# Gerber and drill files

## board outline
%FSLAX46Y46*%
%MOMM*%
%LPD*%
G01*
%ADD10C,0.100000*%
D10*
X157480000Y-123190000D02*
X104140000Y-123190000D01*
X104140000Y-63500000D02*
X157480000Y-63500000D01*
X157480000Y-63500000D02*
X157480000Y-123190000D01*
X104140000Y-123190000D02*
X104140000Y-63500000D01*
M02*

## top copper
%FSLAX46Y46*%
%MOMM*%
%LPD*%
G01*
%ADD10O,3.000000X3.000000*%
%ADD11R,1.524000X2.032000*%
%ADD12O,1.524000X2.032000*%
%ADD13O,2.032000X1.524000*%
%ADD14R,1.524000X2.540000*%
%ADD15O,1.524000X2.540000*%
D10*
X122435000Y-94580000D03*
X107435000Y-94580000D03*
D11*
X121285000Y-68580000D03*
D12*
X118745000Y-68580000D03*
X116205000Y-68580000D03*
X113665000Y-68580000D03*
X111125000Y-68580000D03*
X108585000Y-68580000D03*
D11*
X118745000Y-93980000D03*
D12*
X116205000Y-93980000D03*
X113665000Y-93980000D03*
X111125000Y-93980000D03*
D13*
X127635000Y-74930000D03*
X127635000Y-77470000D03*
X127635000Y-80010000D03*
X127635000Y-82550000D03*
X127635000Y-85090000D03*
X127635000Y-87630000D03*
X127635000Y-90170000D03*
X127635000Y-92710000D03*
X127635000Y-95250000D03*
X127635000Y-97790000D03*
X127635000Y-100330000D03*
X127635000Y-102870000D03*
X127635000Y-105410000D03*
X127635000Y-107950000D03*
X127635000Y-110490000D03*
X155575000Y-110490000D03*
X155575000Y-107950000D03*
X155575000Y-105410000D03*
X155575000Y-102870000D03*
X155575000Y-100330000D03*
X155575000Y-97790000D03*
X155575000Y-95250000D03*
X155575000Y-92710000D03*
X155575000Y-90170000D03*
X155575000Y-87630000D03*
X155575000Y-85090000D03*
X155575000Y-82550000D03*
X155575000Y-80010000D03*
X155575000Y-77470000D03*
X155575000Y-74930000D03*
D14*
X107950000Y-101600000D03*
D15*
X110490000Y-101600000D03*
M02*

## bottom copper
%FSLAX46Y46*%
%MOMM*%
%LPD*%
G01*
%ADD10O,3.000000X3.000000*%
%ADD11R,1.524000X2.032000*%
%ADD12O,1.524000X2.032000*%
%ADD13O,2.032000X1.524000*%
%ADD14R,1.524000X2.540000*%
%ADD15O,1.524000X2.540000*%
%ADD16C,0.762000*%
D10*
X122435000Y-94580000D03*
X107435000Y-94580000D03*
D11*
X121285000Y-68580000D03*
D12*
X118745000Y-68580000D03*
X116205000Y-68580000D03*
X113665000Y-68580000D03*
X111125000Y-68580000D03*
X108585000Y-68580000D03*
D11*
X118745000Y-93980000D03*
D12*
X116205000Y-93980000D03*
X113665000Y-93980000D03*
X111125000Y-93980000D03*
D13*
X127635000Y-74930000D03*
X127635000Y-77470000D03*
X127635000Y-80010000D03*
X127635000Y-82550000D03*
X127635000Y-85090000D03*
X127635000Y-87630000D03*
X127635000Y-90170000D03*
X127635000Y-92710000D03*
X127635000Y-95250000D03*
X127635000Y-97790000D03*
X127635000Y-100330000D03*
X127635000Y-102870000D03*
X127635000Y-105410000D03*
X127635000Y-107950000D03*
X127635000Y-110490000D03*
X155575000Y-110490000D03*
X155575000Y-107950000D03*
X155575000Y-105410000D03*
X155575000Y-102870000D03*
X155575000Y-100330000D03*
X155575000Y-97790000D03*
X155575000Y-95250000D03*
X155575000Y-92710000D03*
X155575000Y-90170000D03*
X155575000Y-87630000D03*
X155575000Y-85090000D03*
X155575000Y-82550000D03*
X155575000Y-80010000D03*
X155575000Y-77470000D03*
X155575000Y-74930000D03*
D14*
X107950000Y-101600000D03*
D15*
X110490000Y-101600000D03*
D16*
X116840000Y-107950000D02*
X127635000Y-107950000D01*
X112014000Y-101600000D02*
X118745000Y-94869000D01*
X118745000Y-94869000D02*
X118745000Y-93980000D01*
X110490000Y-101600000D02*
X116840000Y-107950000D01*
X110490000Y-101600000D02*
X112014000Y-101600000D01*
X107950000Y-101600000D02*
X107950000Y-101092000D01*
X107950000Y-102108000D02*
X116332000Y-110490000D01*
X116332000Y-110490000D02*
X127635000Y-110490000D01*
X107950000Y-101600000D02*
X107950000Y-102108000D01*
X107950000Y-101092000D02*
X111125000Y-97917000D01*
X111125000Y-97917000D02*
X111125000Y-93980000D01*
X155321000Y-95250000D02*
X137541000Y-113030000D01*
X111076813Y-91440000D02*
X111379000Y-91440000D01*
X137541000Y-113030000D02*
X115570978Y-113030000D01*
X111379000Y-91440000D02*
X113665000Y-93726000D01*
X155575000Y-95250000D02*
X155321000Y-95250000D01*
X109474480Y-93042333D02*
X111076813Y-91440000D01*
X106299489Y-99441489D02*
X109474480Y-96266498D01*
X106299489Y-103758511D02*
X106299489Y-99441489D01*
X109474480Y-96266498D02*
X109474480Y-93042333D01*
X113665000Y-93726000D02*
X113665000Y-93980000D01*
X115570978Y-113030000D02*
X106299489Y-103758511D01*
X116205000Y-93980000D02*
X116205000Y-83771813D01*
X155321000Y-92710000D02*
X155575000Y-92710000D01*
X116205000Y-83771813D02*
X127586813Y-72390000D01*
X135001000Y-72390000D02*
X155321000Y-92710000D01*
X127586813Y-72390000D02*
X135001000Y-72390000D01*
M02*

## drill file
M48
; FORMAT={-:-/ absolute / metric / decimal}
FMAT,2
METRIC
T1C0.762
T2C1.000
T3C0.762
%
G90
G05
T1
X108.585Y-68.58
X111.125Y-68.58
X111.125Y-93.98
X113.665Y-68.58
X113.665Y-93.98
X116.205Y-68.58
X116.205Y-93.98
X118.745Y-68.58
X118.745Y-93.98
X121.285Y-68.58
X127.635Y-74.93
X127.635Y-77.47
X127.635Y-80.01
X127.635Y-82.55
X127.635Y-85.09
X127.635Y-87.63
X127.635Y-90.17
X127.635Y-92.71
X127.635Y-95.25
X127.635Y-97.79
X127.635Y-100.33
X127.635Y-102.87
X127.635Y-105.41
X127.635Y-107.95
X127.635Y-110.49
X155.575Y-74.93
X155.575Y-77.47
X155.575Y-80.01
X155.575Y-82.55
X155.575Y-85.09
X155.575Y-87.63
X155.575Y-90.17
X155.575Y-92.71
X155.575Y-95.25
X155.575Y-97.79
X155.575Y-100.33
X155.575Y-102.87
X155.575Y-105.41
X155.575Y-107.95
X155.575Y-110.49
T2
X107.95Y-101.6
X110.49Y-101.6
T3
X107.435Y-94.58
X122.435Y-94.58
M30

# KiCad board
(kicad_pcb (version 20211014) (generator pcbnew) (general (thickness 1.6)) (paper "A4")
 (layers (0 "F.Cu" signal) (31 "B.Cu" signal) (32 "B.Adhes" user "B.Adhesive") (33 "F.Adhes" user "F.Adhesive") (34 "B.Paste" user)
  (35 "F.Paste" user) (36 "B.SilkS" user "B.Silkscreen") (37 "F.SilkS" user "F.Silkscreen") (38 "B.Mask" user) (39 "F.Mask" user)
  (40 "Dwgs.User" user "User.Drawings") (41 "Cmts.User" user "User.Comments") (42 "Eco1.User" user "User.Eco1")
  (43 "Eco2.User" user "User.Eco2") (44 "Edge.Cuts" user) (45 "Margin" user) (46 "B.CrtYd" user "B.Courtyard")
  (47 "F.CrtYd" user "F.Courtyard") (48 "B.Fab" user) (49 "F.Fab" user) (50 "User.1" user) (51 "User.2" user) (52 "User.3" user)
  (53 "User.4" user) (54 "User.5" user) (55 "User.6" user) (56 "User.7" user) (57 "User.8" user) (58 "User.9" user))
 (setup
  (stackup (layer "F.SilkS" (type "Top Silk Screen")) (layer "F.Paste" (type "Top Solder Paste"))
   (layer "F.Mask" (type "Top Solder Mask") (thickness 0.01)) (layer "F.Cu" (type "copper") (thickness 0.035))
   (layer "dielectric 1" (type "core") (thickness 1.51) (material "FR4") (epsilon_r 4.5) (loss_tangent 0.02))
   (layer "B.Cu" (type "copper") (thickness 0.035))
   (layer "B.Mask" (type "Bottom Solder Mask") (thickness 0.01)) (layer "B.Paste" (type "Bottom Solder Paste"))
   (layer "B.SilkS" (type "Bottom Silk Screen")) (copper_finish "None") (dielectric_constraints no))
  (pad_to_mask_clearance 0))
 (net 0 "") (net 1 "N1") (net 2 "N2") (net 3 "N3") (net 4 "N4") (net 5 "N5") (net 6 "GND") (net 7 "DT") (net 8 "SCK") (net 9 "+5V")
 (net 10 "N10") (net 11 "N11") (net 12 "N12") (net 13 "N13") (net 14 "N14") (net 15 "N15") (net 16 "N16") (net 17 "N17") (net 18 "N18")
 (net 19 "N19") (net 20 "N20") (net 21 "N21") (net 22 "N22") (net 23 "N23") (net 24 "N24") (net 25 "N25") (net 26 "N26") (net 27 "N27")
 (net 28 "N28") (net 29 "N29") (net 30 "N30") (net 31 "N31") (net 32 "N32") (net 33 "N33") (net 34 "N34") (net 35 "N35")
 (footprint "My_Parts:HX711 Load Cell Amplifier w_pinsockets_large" (layer "F.Cu") (at 114.935 68.58 -90)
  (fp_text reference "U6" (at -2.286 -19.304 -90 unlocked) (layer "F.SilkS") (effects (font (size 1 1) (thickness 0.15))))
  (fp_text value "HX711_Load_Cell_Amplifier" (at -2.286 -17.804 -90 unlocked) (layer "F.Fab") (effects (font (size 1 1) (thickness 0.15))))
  (pad "" np_thru_hole oval (at 26 -7.5 270) (size 3 3) (drill 0.762) (layers F&B.Cu *.Mask))
  (pad "" np_thru_hole oval (at 26 7.5 270) (size 3 3) (drill 0.762) (layers F&B.Cu *.Mask))
  (pad "1" thru_hole rect (at 0 -6.35 270) (size 2.032 1.524) (drill 0.762) (layers *.Cu *.Mask) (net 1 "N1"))
  (pad "2" thru_hole oval (at 0 -3.81 270) (size 2.032 1.524) (drill 0.762) (layers *.Cu *.Mask) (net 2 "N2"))
  (pad "3" thru_hole oval (at 0 -1.27 270) (size 2.032 1.524) (drill 0.762) (layers *.Cu *.Mask))
  (pad "4" thru_hole oval (at 0 1.27 270) (size 2.032 1.524) (drill 0.762) (layers *.Cu *.Mask) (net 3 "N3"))
  (pad "5" thru_hole oval (at 0 3.81 270) (size 2.032 1.524) (drill 0.762) (layers *.Cu *.Mask) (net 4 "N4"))
  (pad "6" thru_hole oval (at 0 6.35 270) (size 2.032 1.524) (drill 0.762) (layers *.Cu *.Mask) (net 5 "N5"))
  (pad "7" thru_hole rect (at 25.4 -3.81 270) (size 2.032 1.524) (drill 0.762) (layers *.Cu *.Mask) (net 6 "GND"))
  (pad "8" thru_hole oval (at 25.4 -1.27 270) (size 2.032 1.524) (drill 0.762) (layers *.Cu *.Mask) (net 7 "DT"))
  (pad "9" thru_hole oval (at 25.4 1.27 270) (size 2.032 1.524) (drill 0.762) (layers *.Cu *.Mask) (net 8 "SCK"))
  (pad "10" thru_hole oval (at 25.4 3.81 270) (size 2.032 1.524) (drill 0.762) (layers *.Cu *.Mask) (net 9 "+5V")))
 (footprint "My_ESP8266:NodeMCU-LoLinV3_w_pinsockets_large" (layer "F.Cu") (at 141.605 95.25)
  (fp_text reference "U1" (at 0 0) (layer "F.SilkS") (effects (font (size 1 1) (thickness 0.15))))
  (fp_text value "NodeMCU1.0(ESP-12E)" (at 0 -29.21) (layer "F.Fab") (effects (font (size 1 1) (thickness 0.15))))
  (pad "1" thru_hole oval (at -13.97 -20.32) (size 2.032 1.524) (drill 0.762) (layers *.Cu *.Mask "F.SilkS") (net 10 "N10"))
  (pad "2" thru_hole oval (at -13.97 -17.78) (size 2.032 1.524) (drill 0.762) (layers *.Cu *.Mask "F.SilkS") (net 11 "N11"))
  (pad "3" thru_hole oval (at -13.97 -15.24) (size 2.032 1.524) (drill 0.762) (layers *.Cu *.Mask "F.SilkS") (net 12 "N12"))
  (pad "4" thru_hole oval (at -13.97 -12.7) (size 2.032 1.524) (drill 0.762) (layers *.Cu *.Mask "F.SilkS") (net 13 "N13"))
  (pad "5" thru_hole oval (at -13.97 -10.16) (size 2.032 1.524) (drill 0.762) (layers *.Cu *.Mask "F.SilkS") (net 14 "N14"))
  (pad "6" thru_hole oval (at -13.97 -7.62) (size 2.032 1.524) (drill 0.762) (layers *.Cu *.Mask "F.SilkS") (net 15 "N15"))
  (pad "7" thru_hole oval (at -13.97 -5.08) (size 2.032 1.524) (drill 0.762) (layers *.Cu *.Mask "F.SilkS") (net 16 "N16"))
  (pad "8" thru_hole oval (at -13.97 -2.54) (size 2.032 1.524) (drill 0.762) (layers *.Cu *.Mask "F.SilkS") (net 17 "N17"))
  (pad "9" thru_hole oval (at -13.97 0) (size 2.032 1.524) (drill 0.762) (layers *.Cu *.Mask "F.SilkS") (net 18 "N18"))
  (pad "10" thru_hole oval (at -13.97 2.54) (size 2.032 1.524) (drill 0.762) (layers *.Cu *.Mask "F.SilkS") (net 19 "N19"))
  (pad "11" thru_hole oval (at -13.97 5.08) (size 2.032 1.524) (drill 0.762) (layers *.Cu *.Mask "F.SilkS") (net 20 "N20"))
  (pad "12" thru_hole oval (at -13.97 7.62) (size 2.032 1.524) (drill 0.762) (layers *.Cu *.Mask "F.SilkS") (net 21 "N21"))
  (pad "13" thru_hole oval (at -13.97 10.16) (size 2.032 1.524) (drill 0.762) (layers *.Cu *.Mask "F.SilkS") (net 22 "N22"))
  (pad "14" thru_hole oval (at -13.97 12.7) (size 2.032 1.524) (drill 0.762) (layers *.Cu *.Mask "F.SilkS") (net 6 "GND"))
  (pad "15" thru_hole oval (at -13.97 15.24) (size 2.032 1.524) (drill 0.762) (layers *.Cu *.Mask "F.SilkS") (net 9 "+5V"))
  (pad "16" thru_hole oval (at 13.97 15.24) (size 2.032 1.524) (drill 0.762) (layers *.Cu *.Mask "F.SilkS") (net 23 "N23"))
  (pad "17" thru_hole oval (at 13.97 12.7) (size 2.032 1.524) (drill 0.762) (layers *.Cu *.Mask "F.SilkS") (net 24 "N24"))
  (pad "18" thru_hole oval (at 13.97 10.16) (size 2.032 1.524) (drill 0.762) (layers *.Cu *.Mask "F.SilkS") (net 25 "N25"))
  (pad "19" thru_hole oval (at 13.97 7.62) (size 2.032 1.524) (drill 0.762) (layers *.Cu *.Mask "F.SilkS") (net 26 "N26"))
  (pad "20" thru_hole oval (at 13.97 5.08) (size 2.032 1.524) (drill 0.762) (layers *.Cu *.Mask "F.SilkS") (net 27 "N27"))
  (pad "21" thru_hole oval (at 13.97 2.54) (size 2.032 1.524) (drill 0.762) (layers *.Cu *.Mask "F.SilkS") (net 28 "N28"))
  (pad "22" thru_hole oval (at 13.97 0) (size 2.032 1.524) (drill 0.762) (layers *.Cu *.Mask "F.SilkS") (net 8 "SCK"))
  (pad "23" thru_hole oval (at 13.97 -2.54) (size 2.032 1.524) (drill 0.762) (layers *.Cu *.Mask "F.SilkS") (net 7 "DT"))
  (pad "24" thru_hole oval (at 13.97 -5.08) (size 2.032 1.524) (drill 0.762) (layers *.Cu *.Mask "F.SilkS") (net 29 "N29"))
  (pad "25" thru_hole oval (at 13.97 -7.62) (size 2.032 1.524) (drill 0.762) (layers *.Cu *.Mask "F.SilkS") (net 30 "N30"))
  (pad "26" thru_hole oval (at 13.97 -10.16) (size 2.032 1.524) (drill 0.762) (layers *.Cu *.Mask "F.SilkS") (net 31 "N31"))
  (pad "27" thru_hole oval (at 13.97 -12.7) (size 2.032 1.524) (drill 0.762) (layers *.Cu *.Mask "F.SilkS") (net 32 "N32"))
  (pad "28" thru_hole oval (at 13.97 -15.24) (size 2.032 1.524) (drill 0.762) (layers *.Cu *.Mask "F.SilkS") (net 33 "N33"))
  (pad "29" thru_hole oval (at 13.97 -17.78) (size 2.032 1.524) (drill 0.762) (layers *.Cu *.Mask "F.SilkS") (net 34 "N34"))
  (pad "30" thru_hole oval (at 13.97 -20.32) (size 2.032 1.524) (drill 0.762) (layers *.Cu *.Mask "F.SilkS") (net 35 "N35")))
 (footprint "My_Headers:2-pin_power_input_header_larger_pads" (layer "F.Cu") (at 107.95 101.6 90)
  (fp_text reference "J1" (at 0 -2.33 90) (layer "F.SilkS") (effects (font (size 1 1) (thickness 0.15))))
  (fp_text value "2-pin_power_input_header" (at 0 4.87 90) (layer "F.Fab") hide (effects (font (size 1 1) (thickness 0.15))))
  (pad "1" thru_hole rect locked (at 0 0 90) (size 2.54 1.524) (drill 1) (layers *.Cu *.Mask) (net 9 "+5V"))
  (pad "2" thru_hole oval locked (at 0 2.54 90) (size 2.54 1.524) (drill 1) (layers *.Cu *.Mask) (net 6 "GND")))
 (gr_line (start 157.48 123.19) (end 104.14 123.19) (layer "Edge.Cuts") (width 0.1))
 (gr_line (start 104.14 63.5) (end 157.48 63.5) (layer "Edge.Cuts") (width 0.1))
 (gr_line (start 157.48 63.5) (end 157.48 123.19) (layer "Edge.Cuts") (width 0.1))
 (gr_line (start 104.14 123.19) (end 104.14 63.5) (layer "Edge.Cuts") (width 0.1))
 (segment (start 116.84 107.95) (end 127.635 107.95) (width 0.762) (layer "B.Cu") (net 6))
 (segment (start 112.014 101.6) (end 118.745 94.869) (width 0.762) (layer "B.Cu") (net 6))
 (segment (start 118.745 94.869) (end 118.745 93.98) (width 0.762) (layer "B.Cu") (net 6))
 (segment (start 110.49 101.6) (end 116.84 107.95) (width 0.762) (layer "B.Cu") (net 6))
 (segment (start 110.49 101.6) (end 112.014 101.6) (width 0.762) (layer "B.Cu") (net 6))
 (segment (start 107.95 101.6) (end 107.95 101.092) (width 0.762) (layer "B.Cu") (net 9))
 (segment (start 107.95 102.108) (end 116.332 110.49) (width 0.762) (layer "B.Cu") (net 9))
 (segment (start 116.332 110.49) (end 127.635 110.49) (width 0.762) (layer "B.Cu") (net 9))
 (segment (start 107.95 101.6) (end 107.95 102.108) (width 0.762) (layer "B.Cu") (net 9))
 (segment (start 107.95 101.092) (end 111.125 97.917) (width 0.762) (layer "B.Cu") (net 9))
 (segment (start 111.125 97.917) (end 111.125 93.98) (width 0.762) (layer "B.Cu") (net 9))
 (segment (start 155.321 95.25) (end 137.541 113.03) (width 0.762) (layer "B.Cu") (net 8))
 (segment (start 111.076813 91.44) (end 111.379 91.44) (width 0.762) (layer "B.Cu") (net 8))
 (segment (start 137.541 113.03) (end 115.570978 113.03) (width 0.762) (layer "B.Cu") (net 8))
 (segment (start 111.379 91.44) (end 113.665 93.726) (width 0.762) (layer "B.Cu") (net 8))
 (segment (start 155.575 95.25) (end 155.321 95.25) (width 0.762) (layer "B.Cu") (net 8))
 (segment (start 109.47448 93.042333) (end 111.076813 91.44) (width 0.762) (layer "B.Cu") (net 8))
 (segment (start 106.299489 99.441489) (end 109.47448 96.266498) (width 0.762) (layer "B.Cu") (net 8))
 (segment (start 106.299489 103.758511) (end 106.299489 99.441489) (width 0.762) (layer "B.Cu") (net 8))
 (segment (start 109.47448 96.266498) (end 109.47448 93.042333) (width 0.762) (layer "B.Cu") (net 8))
 (segment (start 113.665 93.726) (end 113.665 93.98) (width 0.762) (layer "B.Cu") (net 8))
 (segment (start 115.570978 113.03) (end 106.299489 103.758511) (width 0.762) (layer "B.Cu") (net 8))
 (segment (start 116.205 93.98) (end 116.205 83.771813) (width 0.762) (layer "B.Cu") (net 7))
 (segment (start 155.321 92.71) (end 155.575 92.71) (width 0.762) (layer "B.Cu") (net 7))
 (segment (start 116.205 83.771813) (end 127.586813 72.39) (width 0.762) (layer "B.Cu") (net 7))
 (segment (start 135.001 72.39) (end 155.321 92.71) (width 0.762) (layer "B.Cu") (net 7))
 (segment (start 127.586813 72.39) (end 135.001 72.39) (width 0.762) (layer "B.Cu") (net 7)))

